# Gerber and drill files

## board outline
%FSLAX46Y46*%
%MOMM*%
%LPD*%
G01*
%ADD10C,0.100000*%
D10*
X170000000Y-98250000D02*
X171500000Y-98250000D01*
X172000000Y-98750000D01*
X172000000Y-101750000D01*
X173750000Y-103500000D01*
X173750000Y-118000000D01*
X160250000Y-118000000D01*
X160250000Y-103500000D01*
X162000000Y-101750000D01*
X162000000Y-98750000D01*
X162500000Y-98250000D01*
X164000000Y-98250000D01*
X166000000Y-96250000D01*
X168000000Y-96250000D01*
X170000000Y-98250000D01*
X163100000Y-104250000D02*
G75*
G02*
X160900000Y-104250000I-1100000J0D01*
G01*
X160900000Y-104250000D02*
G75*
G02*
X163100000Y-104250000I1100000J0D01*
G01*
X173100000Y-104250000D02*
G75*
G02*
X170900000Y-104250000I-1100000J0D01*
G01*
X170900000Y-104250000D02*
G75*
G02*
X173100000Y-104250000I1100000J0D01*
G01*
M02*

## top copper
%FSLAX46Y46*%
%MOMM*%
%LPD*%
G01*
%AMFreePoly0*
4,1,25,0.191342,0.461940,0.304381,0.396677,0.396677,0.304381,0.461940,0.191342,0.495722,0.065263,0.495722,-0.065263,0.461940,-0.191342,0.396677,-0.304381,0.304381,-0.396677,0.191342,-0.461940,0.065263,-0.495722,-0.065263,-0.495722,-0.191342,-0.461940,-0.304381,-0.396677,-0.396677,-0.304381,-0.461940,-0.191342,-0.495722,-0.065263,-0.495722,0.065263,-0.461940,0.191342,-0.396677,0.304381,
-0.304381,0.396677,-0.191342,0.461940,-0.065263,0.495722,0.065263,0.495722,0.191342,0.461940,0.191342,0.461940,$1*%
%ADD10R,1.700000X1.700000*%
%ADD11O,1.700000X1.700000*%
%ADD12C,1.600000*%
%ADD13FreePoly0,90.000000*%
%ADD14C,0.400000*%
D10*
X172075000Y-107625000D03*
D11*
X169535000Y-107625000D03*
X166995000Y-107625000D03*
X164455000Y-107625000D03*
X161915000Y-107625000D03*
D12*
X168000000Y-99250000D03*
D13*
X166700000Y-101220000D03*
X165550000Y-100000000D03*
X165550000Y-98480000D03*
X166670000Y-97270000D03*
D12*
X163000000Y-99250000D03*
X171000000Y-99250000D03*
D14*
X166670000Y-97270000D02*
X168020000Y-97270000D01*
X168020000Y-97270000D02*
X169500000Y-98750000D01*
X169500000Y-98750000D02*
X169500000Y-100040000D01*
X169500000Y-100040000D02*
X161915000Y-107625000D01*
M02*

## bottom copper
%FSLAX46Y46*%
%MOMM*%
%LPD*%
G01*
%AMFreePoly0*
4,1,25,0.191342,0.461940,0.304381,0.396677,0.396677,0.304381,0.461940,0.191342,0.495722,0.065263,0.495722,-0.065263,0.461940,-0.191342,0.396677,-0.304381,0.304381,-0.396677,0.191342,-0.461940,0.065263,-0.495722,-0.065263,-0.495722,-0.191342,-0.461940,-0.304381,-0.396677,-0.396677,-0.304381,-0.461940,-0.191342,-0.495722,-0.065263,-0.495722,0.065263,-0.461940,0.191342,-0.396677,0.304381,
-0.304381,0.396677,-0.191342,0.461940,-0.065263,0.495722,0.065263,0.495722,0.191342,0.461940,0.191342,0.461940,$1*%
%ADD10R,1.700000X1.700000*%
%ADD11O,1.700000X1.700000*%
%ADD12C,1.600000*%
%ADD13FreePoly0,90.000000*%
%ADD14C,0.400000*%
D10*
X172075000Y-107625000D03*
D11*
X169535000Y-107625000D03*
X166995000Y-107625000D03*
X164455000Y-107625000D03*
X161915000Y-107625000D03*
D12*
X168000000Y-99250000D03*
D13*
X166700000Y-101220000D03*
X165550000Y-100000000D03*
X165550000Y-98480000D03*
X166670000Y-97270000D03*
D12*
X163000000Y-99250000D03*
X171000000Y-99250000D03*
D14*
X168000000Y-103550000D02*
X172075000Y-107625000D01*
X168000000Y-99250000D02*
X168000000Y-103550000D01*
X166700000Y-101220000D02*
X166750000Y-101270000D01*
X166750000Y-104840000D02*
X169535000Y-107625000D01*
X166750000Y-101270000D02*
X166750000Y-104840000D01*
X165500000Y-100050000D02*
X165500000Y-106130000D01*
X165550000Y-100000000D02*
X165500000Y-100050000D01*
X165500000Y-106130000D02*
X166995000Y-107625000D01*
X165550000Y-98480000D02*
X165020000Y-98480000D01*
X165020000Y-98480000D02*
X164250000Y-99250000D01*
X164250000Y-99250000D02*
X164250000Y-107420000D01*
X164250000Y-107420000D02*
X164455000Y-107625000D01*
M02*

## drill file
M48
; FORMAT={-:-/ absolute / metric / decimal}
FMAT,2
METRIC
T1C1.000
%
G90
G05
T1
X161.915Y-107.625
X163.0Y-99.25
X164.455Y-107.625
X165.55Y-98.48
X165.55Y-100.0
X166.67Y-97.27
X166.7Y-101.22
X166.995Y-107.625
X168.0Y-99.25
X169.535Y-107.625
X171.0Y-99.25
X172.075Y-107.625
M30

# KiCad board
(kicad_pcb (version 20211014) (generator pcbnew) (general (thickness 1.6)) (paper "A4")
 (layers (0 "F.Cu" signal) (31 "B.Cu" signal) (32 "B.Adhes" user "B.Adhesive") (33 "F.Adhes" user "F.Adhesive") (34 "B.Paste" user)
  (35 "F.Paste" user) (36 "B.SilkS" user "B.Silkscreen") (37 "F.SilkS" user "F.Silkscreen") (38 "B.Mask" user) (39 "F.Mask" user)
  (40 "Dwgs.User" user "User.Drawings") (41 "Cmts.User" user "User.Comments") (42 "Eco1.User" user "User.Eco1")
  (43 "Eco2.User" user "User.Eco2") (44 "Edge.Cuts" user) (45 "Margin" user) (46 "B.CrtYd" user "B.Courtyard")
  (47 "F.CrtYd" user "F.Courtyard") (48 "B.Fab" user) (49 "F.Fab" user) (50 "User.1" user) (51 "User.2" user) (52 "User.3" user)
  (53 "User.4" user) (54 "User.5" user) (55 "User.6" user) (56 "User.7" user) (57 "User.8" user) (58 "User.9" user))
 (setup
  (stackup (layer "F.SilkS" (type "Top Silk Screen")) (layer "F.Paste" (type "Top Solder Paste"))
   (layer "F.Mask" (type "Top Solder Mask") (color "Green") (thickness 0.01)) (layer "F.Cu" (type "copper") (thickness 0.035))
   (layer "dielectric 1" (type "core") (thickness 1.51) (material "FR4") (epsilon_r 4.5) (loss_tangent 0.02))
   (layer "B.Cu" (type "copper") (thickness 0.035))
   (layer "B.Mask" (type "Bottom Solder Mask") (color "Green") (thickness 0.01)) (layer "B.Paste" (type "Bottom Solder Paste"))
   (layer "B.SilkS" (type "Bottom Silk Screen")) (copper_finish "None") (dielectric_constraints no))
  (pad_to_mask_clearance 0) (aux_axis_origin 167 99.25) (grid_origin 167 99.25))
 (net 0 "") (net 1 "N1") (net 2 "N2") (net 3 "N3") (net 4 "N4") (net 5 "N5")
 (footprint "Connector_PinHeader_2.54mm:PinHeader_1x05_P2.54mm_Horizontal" (layer "F.Cu") (at 172.075 107.625 -90)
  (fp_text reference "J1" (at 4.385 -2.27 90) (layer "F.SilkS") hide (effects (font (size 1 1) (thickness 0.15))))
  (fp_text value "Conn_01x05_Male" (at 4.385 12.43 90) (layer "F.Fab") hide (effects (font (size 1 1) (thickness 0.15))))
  (pad "1" thru_hole rect (at 0 0 270) (size 1.7 1.7) (drill 1) (layers *.Cu *.Mask) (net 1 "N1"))
  (pad "2" thru_hole oval (at 0 2.54 270) (size 1.7 1.7) (drill 1) (layers *.Cu *.Mask) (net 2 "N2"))
  (pad "3" thru_hole oval (at 0 5.08 270) (size 1.7 1.7) (drill 1) (layers *.Cu *.Mask) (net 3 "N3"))
  (pad "4" thru_hole oval (at 0 7.62 270) (size 1.7 1.7) (drill 1) (layers *.Cu *.Mask) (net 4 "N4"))
  (pad "5" thru_hole oval (at 0 10.16 270) (size 1.7 1.7) (drill 1) (layers *.Cu *.Mask) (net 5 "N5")))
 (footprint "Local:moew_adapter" (layer "F.Cu") (at 167 99.25 90)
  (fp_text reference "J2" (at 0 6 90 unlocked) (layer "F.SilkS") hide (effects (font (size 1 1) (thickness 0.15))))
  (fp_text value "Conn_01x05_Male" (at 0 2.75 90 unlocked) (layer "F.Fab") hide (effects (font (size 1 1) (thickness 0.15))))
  (pad "1" thru_hole circle (at 0 1 90) (size 1.6 1.6) (drill 1) (layers *.Cu *.Mask) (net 1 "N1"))
  (pad "2" thru_hole custom (at -1.97 -0.3 90) (size 1 1) (drill 1) (layers *.Cu *.Mask) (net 2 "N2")
   (options (clearance outline) (anchor circle)) (primitives))
  (pad "3" thru_hole custom (at -0.75 -1.45 90) (size 1 1) (drill 1) (layers *.Cu *.Mask) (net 3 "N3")
   (options (clearance outline) (anchor circle)) (primitives))
  (pad "4" thru_hole custom (at 0.77 -1.45 90) (size 1 1) (drill 1) (layers *.Cu *.Mask) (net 4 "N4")
   (options (clearance outline) (anchor circle)) (primitives))
  (pad "5" thru_hole custom (at 1.98 -0.33 90) (size 1 1) (drill 1) (layers *.Cu *.Mask) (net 5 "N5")
   (options (clearance outline) (anchor circle)) (primitives))
  (pad "NC" thru_hole circle (at 0 -4 90) (size 1.6 1.6) (drill 1) (layers *.Cu *.Mask))
  (pad "NC" thru_hole circle (at 0 4 90) (size 1.6 1.6) (drill 1) (layers *.Cu *.Mask)))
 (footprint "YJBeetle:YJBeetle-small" (layer "B.Cu") (at 167 116.5 180)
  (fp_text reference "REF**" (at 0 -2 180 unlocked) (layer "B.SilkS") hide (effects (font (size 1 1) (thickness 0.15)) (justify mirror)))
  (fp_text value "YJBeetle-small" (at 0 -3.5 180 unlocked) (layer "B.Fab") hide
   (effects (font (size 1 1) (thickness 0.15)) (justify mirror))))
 (gr_poly
  (pts (xy 170 98.25) (xy 171.5 98.25) (xy 172 98.75) (xy 172 101.75) (xy 173.75 103.5) (xy 173.75 118) (xy 160.25 118) (xy 160.25 103.5)
   (xy 162 101.75) (xy 162 98.75) (xy 162.5 98.25) (xy 164 98.25) (xy 166 96.25) (xy 168 96.25))
  (layer "Edge.Cuts") (width 0.1) (fill none))
 (gr_circle (center 162 104.25) (end 163.1 104.25) (layer "Edge.Cuts") (width 0.1) (fill none))
 (gr_circle (center 172 104.25) (end 173.1 104.25) (layer "Edge.Cuts") (width 0.1) (fill none))
 (segment (start 168 103.55) (end 172.075 107.625) (width 0.4) (layer "B.Cu") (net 1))
 (segment (start 168 99.25) (end 168 103.55) (width 0.4) (layer "B.Cu") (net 1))
 (segment (start 166.7 101.22) (end 166.75 101.27) (width 0.4) (layer "B.Cu") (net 2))
 (segment (start 166.75 104.84) (end 169.535 107.625) (width 0.4) (layer "B.Cu") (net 2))
 (segment (start 166.75 101.27) (end 166.75 104.84) (width 0.4) (layer "B.Cu") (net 2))
 (segment (start 165.5 100.05) (end 165.5 106.13) (width 0.4) (layer "B.Cu") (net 3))
 (segment (start 165.55 100) (end 165.5 100.05) (width 0.4) (layer "B.Cu") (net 3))
 (segment (start 165.5 106.13) (end 166.995 107.625) (width 0.4) (layer "B.Cu") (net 3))
 (segment (start 165.55 98.48) (end 165.02 98.48) (width 0.4) (layer "B.Cu") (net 4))
 (segment (start 165.02 98.48) (end 164.25 99.25) (width 0.4) (layer "B.Cu") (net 4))
 (segment (start 164.25 99.25) (end 164.25 107.42) (width 0.4) (layer "B.Cu") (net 4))
 (segment (start 164.25 107.42) (end 164.455 107.625) (width 0.4) (layer "B.Cu") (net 4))
 (segment (start 166.67 97.27) (end 168.02 97.27) (width 0.4) (layer "F.Cu") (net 5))
 (segment (start 168.02 97.27) (end 169.5 98.75) (width 0.4) (layer "F.Cu") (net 5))
 (segment (start 169.5 98.75) (end 169.5 100.04) (width 0.4) (layer "F.Cu") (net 5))
 (segment (start 169.5 100.04) (end 161.915 107.625) (width 0.4) (layer "F.Cu") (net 5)))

